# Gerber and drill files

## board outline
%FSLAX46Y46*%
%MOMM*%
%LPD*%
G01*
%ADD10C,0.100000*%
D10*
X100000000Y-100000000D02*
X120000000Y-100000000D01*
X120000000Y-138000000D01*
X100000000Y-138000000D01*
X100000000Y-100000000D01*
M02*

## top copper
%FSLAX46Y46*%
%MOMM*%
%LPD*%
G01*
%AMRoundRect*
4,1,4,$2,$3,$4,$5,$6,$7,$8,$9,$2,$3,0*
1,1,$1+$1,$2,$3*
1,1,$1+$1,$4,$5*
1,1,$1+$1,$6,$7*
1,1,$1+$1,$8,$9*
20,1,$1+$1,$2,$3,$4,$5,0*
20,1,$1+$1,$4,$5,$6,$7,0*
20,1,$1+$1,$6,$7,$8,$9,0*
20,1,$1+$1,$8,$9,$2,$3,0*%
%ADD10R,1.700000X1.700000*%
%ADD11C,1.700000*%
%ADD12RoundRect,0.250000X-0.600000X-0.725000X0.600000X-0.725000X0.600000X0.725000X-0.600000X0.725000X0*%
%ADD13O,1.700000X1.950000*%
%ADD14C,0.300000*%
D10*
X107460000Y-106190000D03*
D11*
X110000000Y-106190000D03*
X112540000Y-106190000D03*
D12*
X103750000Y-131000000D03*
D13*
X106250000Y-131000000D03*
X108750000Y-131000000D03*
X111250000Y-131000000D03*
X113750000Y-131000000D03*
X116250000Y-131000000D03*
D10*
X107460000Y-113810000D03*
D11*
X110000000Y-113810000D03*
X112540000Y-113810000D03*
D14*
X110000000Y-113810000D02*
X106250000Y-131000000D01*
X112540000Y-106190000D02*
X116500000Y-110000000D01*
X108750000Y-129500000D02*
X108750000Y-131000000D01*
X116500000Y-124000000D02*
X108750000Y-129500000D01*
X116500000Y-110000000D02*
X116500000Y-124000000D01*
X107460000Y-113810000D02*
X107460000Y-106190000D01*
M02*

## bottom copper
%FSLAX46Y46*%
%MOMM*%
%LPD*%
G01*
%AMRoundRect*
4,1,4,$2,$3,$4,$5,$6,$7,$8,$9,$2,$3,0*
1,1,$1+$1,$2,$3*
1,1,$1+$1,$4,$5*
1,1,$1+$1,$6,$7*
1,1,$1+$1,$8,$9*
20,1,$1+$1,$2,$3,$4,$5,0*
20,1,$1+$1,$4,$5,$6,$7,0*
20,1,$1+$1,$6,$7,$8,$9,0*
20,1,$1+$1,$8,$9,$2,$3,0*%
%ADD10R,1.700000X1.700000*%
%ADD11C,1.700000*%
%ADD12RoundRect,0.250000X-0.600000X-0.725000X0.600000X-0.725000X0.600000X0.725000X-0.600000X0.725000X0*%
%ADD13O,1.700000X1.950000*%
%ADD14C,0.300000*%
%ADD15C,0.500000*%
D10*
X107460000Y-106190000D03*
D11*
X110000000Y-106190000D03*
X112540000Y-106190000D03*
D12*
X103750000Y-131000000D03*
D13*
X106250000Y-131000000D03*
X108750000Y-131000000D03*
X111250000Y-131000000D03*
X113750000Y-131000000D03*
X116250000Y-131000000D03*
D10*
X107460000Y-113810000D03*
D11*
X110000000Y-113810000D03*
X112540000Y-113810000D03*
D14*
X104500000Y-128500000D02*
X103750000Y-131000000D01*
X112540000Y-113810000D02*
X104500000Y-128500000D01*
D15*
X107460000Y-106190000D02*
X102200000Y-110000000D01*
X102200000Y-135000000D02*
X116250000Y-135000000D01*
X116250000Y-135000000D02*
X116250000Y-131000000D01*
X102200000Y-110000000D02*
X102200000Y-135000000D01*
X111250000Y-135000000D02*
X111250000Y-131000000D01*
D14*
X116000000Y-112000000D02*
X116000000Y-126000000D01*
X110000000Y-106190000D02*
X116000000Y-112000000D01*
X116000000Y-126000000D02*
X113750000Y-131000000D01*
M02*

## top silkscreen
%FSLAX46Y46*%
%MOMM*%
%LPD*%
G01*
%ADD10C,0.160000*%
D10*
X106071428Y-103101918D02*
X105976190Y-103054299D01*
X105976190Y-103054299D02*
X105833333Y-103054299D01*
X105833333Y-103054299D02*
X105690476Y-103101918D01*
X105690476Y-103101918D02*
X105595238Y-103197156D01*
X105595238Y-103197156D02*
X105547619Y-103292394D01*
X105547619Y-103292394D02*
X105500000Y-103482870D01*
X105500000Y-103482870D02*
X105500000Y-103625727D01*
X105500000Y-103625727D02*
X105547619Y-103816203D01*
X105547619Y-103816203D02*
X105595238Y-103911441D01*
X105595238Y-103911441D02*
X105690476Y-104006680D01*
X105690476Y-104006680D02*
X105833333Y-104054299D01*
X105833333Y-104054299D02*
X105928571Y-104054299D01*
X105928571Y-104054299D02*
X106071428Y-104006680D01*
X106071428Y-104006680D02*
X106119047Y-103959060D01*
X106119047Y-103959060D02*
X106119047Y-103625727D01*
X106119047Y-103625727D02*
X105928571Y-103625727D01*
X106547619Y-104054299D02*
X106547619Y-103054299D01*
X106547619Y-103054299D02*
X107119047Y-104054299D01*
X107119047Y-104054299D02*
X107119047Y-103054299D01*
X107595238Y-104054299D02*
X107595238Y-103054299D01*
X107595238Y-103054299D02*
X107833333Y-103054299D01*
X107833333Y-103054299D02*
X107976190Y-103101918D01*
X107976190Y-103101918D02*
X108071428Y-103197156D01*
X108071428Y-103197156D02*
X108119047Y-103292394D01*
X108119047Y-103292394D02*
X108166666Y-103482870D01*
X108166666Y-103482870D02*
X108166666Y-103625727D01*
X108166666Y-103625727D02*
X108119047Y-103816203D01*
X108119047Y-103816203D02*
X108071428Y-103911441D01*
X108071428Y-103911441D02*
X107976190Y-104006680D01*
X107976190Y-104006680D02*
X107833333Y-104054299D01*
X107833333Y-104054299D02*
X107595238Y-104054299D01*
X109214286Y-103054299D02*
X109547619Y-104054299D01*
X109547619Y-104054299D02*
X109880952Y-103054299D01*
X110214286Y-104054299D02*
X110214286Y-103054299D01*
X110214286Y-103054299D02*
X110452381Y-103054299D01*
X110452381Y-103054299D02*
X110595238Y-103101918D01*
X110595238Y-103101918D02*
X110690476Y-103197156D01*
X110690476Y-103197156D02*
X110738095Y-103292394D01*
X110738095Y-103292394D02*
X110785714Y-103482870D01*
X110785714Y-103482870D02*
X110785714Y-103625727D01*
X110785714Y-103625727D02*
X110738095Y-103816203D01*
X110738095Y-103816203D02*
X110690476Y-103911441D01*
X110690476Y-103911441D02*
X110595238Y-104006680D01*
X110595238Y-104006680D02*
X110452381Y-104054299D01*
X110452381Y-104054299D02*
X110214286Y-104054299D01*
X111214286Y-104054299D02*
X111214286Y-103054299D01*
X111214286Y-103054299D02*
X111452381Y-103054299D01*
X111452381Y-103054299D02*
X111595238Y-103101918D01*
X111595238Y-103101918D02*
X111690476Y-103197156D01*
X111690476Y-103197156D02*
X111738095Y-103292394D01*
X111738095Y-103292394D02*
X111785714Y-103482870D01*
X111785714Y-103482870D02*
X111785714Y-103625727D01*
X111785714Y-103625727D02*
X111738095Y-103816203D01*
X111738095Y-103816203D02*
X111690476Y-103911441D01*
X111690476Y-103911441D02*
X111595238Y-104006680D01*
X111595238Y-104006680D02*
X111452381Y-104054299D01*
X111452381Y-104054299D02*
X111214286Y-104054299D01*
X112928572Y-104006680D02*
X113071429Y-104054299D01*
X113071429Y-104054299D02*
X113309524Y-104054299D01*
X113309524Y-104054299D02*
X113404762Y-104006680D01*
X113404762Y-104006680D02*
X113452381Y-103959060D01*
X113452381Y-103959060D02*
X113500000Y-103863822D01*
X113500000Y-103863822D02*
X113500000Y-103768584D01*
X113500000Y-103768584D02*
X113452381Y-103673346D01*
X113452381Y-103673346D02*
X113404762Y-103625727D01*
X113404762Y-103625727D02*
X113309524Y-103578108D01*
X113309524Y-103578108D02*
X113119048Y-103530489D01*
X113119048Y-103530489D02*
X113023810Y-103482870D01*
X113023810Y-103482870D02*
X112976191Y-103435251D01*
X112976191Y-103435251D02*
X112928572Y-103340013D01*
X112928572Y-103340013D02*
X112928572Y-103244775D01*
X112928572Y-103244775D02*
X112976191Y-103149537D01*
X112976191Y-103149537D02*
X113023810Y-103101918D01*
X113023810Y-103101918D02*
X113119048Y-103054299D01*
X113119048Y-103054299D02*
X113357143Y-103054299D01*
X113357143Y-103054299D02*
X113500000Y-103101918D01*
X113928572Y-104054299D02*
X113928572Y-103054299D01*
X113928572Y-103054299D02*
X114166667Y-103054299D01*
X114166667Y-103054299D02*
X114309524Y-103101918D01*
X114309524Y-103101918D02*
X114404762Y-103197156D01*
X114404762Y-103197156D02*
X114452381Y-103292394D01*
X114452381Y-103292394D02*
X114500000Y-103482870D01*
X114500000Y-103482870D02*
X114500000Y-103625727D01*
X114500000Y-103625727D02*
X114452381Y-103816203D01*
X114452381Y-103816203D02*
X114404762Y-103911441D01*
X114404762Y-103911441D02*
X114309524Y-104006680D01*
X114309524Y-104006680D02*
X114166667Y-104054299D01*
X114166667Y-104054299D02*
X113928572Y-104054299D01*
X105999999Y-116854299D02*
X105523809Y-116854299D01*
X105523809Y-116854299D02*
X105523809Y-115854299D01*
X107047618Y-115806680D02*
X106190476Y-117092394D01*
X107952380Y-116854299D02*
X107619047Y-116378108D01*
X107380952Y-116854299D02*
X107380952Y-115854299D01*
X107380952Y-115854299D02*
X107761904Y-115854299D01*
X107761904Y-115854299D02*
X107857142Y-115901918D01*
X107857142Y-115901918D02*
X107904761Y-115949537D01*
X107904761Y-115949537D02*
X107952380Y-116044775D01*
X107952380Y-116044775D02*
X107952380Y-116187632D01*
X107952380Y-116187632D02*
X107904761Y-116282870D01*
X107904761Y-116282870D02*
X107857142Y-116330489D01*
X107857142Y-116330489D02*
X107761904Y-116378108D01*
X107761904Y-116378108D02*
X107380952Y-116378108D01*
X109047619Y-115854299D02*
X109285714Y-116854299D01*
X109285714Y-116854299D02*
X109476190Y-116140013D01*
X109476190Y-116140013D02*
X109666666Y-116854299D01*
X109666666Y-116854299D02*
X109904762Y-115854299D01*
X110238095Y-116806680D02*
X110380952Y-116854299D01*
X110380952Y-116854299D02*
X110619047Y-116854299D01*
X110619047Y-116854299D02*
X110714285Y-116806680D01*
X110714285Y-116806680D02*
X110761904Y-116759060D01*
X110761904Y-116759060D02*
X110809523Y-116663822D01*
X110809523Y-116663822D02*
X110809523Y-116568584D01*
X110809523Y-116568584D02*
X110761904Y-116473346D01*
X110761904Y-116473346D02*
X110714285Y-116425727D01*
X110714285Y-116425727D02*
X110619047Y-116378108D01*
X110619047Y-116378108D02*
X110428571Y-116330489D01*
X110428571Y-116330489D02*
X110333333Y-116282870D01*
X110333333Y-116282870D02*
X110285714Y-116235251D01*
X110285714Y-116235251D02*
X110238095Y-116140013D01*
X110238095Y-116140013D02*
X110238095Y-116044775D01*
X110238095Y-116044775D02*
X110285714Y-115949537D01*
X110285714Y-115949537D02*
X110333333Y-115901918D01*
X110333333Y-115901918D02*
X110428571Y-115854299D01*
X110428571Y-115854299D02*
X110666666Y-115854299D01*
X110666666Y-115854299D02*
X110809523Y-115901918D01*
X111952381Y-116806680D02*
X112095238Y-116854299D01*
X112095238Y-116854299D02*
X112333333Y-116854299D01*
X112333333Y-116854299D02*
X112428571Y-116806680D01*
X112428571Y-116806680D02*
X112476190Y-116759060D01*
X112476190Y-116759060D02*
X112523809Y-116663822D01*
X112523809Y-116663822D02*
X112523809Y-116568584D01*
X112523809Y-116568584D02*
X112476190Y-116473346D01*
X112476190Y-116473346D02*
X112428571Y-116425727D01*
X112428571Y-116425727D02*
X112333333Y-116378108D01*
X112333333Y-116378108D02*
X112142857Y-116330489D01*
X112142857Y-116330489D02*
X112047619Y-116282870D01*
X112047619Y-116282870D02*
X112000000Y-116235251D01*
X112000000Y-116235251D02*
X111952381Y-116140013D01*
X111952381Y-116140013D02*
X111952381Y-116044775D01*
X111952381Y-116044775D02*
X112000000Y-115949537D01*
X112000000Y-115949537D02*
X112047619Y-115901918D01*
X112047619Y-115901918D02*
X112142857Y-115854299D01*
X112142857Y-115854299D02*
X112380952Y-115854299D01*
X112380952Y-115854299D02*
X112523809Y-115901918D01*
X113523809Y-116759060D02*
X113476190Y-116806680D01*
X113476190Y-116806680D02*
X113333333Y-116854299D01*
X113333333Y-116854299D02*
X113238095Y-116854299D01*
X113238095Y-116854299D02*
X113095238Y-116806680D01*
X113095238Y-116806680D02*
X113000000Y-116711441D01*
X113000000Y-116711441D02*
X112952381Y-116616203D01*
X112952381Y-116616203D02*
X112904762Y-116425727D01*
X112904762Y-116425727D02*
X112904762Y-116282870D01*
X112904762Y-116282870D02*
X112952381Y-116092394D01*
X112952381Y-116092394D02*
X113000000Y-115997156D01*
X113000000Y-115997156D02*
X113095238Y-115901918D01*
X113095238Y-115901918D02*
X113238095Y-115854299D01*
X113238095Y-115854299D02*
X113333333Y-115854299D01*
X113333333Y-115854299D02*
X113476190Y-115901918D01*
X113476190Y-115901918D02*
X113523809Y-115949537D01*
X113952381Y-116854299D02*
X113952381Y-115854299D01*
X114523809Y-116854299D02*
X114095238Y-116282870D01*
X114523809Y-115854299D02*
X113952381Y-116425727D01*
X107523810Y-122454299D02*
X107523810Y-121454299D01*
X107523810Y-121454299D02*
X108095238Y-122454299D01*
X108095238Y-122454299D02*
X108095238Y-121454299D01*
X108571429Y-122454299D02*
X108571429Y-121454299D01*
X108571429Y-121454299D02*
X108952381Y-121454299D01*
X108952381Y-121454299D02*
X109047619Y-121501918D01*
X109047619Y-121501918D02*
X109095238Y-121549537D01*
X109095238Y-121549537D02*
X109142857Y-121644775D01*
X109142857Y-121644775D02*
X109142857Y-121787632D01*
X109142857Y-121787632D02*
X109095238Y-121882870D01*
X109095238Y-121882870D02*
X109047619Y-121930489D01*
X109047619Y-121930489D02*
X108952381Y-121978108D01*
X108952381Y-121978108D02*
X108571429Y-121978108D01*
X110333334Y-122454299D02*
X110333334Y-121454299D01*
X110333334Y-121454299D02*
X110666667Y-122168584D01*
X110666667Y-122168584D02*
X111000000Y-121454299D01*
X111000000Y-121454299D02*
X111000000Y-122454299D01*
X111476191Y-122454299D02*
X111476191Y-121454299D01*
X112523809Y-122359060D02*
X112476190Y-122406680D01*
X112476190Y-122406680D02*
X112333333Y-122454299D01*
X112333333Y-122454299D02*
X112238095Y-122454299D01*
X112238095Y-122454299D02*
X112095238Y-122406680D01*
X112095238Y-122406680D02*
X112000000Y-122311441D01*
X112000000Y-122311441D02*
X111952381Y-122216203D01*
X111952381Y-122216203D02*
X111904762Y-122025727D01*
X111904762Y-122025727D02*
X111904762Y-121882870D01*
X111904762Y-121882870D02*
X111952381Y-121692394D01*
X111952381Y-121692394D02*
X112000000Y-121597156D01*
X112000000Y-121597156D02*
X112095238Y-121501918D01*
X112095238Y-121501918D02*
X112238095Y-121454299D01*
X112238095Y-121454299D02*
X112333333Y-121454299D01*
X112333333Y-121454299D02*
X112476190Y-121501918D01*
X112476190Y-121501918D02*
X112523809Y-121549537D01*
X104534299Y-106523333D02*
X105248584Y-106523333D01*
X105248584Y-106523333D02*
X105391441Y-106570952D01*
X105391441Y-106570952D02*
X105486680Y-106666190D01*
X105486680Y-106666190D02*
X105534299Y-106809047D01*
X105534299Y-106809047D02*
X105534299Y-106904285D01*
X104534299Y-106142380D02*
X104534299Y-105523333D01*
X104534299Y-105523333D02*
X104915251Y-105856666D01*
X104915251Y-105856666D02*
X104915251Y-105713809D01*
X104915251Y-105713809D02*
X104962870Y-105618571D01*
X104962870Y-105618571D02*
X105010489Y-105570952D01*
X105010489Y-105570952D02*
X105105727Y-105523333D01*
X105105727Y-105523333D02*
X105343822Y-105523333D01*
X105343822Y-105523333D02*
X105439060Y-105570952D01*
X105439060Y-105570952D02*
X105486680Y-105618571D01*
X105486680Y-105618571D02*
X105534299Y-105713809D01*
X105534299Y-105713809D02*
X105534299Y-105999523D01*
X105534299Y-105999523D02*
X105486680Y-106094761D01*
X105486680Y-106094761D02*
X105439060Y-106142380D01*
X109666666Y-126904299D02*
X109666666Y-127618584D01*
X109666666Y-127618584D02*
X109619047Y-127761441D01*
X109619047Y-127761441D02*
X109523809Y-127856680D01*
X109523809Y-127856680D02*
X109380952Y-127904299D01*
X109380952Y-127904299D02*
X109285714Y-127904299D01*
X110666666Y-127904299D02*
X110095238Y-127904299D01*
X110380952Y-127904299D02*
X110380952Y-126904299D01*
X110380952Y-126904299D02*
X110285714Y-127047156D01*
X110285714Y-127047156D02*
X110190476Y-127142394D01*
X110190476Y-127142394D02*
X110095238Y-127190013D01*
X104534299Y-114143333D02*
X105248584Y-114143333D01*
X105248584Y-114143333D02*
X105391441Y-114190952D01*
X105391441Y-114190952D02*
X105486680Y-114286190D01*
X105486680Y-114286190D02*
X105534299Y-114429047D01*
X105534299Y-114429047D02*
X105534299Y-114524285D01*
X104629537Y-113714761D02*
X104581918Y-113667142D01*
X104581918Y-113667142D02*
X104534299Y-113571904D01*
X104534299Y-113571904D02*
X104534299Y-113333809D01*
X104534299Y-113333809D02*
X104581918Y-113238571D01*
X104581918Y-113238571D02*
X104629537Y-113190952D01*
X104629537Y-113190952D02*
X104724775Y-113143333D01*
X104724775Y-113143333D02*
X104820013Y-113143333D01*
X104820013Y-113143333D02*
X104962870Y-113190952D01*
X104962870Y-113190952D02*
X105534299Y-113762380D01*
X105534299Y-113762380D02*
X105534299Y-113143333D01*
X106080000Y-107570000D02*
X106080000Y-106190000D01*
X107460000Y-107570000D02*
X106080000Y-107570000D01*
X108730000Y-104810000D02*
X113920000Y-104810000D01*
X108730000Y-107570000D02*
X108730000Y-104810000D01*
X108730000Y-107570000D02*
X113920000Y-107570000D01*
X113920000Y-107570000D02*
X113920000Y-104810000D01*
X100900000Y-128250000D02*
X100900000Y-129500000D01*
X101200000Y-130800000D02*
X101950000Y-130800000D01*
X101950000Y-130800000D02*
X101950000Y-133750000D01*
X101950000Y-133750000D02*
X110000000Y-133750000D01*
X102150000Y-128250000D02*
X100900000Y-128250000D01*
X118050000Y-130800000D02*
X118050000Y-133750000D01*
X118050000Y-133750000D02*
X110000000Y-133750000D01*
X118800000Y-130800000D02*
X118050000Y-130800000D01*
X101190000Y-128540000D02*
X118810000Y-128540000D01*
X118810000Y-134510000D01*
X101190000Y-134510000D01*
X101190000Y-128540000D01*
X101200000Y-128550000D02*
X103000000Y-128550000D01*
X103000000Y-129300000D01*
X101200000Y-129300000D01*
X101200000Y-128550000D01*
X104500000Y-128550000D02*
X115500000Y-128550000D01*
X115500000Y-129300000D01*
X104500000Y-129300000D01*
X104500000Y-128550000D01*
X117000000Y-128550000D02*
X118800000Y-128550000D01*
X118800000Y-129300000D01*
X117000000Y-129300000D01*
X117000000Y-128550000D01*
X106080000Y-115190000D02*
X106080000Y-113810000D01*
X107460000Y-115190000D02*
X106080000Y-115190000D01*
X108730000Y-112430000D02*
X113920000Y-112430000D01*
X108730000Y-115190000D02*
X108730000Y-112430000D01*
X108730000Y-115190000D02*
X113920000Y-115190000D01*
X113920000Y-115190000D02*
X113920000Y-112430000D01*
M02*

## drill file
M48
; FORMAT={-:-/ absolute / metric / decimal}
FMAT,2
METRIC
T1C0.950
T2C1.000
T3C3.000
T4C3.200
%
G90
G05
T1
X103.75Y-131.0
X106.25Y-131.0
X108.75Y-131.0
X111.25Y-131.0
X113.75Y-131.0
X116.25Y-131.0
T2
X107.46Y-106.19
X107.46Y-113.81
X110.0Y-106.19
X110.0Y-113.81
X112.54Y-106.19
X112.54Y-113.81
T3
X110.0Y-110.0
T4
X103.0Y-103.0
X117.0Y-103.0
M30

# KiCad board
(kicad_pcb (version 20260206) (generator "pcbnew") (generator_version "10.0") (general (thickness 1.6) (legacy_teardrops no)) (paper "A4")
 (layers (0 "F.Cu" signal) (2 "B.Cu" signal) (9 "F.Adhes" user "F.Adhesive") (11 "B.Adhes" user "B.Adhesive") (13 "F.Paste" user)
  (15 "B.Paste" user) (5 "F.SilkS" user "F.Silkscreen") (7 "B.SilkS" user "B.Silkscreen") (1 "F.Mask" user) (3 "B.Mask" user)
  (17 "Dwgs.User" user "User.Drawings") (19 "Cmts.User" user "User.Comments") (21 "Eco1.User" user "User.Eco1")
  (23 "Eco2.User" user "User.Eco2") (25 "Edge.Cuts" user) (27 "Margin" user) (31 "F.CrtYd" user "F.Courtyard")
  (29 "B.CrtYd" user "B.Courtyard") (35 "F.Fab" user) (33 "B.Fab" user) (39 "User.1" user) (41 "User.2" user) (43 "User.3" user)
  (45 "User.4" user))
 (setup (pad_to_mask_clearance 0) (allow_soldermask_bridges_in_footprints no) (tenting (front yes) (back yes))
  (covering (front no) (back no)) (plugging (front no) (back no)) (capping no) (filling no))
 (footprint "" (layer "F.Cu") (at 110 110)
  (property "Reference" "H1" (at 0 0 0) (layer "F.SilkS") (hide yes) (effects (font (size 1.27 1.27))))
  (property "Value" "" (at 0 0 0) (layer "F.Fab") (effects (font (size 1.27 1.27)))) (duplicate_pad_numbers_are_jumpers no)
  (pad "" np_thru_hole circle (at 0 0) (size 3 3) (drill 3) (layers "*.Cu" "*.Mask")))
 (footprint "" (layer "F.Cu") (at 117 103)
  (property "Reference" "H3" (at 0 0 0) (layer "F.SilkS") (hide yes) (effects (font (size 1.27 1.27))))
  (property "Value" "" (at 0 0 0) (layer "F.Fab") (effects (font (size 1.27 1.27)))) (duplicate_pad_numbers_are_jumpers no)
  (pad "" np_thru_hole circle (at 0 0) (size 3.2 3.2) (drill 3.2) (layers "*.Cu" "*.Mask")))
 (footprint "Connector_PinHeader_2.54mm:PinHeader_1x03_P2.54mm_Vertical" (layer "F.Cu") (at 107.46 106.19 90)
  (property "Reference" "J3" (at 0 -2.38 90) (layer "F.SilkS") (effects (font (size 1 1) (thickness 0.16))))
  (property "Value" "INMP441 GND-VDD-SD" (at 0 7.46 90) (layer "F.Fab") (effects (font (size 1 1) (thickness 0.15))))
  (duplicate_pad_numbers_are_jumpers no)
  (fp_line (start -1.38 -1.38) (end 0 -1.38) (stroke (width 0.16) (type solid)) (layer "F.SilkS"))
  (fp_line (start -1.38 0) (end -1.38 -1.38) (stroke (width 0.16) (type solid)) (layer "F.SilkS"))
  (fp_line (start 1.38 1.27) (end 1.38 6.46) (stroke (width 0.16) (type solid)) (layer "F.SilkS"))
  (fp_line (start -1.38 1.27) (end 1.38 1.27) (stroke (width 0.16) (type solid)) (layer "F.SilkS"))
  (fp_line (start -1.38 1.27) (end -1.38 6.46) (stroke (width 0.16) (type solid)) (layer "F.SilkS"))
  (fp_line (start -1.38 6.46) (end 1.38 6.46) (stroke (width 0.16) (type solid)) (layer "F.SilkS"))
  (pad "1" thru_hole rect (at 0 0 90) (size 1.7 1.7) (drill 1) (layers "*.Cu" "*.Mask") (remove_unused_layers no) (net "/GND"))
  (pad "2" thru_hole circle (at 0 2.54 90) (size 1.7 1.7) (drill 1) (layers "*.Cu" "*.Mask") (remove_unused_layers no) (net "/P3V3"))
  (pad "3" thru_hole circle (at 0 5.08 90) (size 1.7 1.7) (drill 1) (layers "*.Cu" "*.Mask") (remove_unused_layers no) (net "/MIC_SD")))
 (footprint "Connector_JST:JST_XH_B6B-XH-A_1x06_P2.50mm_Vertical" (layer "F.Cu") (at 103.75 131)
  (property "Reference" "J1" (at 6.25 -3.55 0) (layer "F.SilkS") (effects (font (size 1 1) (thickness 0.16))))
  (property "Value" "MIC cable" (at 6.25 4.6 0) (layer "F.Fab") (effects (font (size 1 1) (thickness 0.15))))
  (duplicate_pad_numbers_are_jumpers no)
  (fp_line (start -2.85 -2.75) (end -2.85 -1.5) (stroke (width 0.16) (type solid)) (layer "F.SilkS"))
  (fp_line (start -2.55 -0.2) (end -1.8 -0.2) (stroke (width 0.16) (type solid)) (layer "F.SilkS"))
  (fp_line (start -1.8 -0.2) (end -1.8 2.75) (stroke (width 0.16) (type solid)) (layer "F.SilkS"))
  (fp_line (start -1.8 2.75) (end 6.25 2.75) (stroke (width 0.16) (type solid)) (layer "F.SilkS"))
  (fp_line (start -1.6 -2.75) (end -2.85 -2.75) (stroke (width 0.16) (type solid)) (layer "F.SilkS"))
  (fp_line (start 14.3 -0.2) (end 14.3 2.75) (stroke (width 0.16) (type solid)) (layer "F.SilkS"))
  (fp_line (start 14.3 2.75) (end 6.25 2.75) (stroke (width 0.16) (type solid)) (layer "F.SilkS"))
  (fp_line (start 15.05 -0.2) (end 14.3 -0.2) (stroke (width 0.16) (type solid)) (layer "F.SilkS"))
  (fp_rect (start -2.56 -2.46) (end 15.06 3.51) (stroke (width 0.16) (type solid)) (fill no) (layer "F.SilkS"))
  (fp_rect (start -2.55 -2.45) (end -0.75 -1.7) (stroke (width 0.16) (type solid)) (fill no) (layer "F.SilkS"))
  (fp_rect (start 0.75 -2.45) (end 11.75 -1.7) (stroke (width 0.16) (type solid)) (fill no) (layer "F.SilkS"))
  (fp_rect (start 13.25 -2.45) (end 15.05 -1.7) (stroke (width 0.16) (type solid)) (fill no) (layer "F.SilkS"))
  (pad "1" thru_hole roundrect (at 0 0) (size 1.7 1.95) (drill 0.95) (layers "*.Cu" "*.Mask") (remove_unused_layers no)
   (roundrect_rratio 0.147059) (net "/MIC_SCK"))
  (pad "2" thru_hole oval (at 2.5 0) (size 1.7 1.95) (drill 0.95) (layers "*.Cu" "*.Mask") (remove_unused_layers no) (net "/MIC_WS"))
  (pad "3" thru_hole oval (at 5 0) (size 1.7 1.95) (drill 0.95) (layers "*.Cu" "*.Mask") (remove_unused_layers no) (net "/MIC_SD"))
  (pad "4" thru_hole oval (at 7.5 0) (size 1.7 1.95) (drill 0.95) (layers "*.Cu" "*.Mask") (remove_unused_layers no) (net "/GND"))
  (pad "5" thru_hole oval (at 10 0) (size 1.7 1.95) (drill 0.95) (layers "*.Cu" "*.Mask") (remove_unused_layers no) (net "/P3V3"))
  (pad "6" thru_hole oval (at 12.5 0) (size 1.7 1.95) (drill 0.95) (layers "*.Cu" "*.Mask") (remove_unused_layers no) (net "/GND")))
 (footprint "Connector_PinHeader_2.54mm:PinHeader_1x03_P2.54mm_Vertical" (layer "F.Cu") (at 107.46 113.81 90)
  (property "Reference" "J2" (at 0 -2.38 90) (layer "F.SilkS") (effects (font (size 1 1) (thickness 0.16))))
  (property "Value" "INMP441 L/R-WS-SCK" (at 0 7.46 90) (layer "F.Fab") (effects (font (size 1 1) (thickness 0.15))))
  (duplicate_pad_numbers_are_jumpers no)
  (fp_line (start -1.38 -1.38) (end 0 -1.38) (stroke (width 0.16) (type solid)) (layer "F.SilkS"))
  (fp_line (start -1.38 0) (end -1.38 -1.38) (stroke (width 0.16) (type solid)) (layer "F.SilkS"))
  (fp_line (start 1.38 1.27) (end 1.38 6.46) (stroke (width 0.16) (type solid)) (layer "F.SilkS"))
  (fp_line (start -1.38 1.27) (end 1.38 1.27) (stroke (width 0.16) (type solid)) (layer "F.SilkS"))
  (fp_line (start -1.38 1.27) (end -1.38 6.46) (stroke (width 0.16) (type solid)) (layer "F.SilkS"))
  (fp_line (start -1.38 6.46) (end 1.38 6.46) (stroke (width 0.16) (type solid)) (layer "F.SilkS"))
  (pad "1" thru_hole rect (at 0 0 90) (size 1.7 1.7) (drill 1) (layers "*.Cu" "*.Mask") (remove_unused_layers no) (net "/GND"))
  (pad "2" thru_hole circle (at 0 2.54 90) (size 1.7 1.7) (drill 1) (layers "*.Cu" "*.Mask") (remove_unused_layers no) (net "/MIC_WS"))
  (pad "3" thru_hole circle (at 0 5.08 90) (size 1.7 1.7) (drill 1) (layers "*.Cu" "*.Mask") (remove_unused_layers no) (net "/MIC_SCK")))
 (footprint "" (layer "F.Cu") (at 103 103)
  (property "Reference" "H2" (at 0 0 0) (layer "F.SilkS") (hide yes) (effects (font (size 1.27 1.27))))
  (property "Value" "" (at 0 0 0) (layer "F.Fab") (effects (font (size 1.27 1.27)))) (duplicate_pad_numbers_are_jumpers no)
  (pad "" np_thru_hole circle (at 0 0) (size 3.2 3.2) (drill 3.2) (layers "*.Cu" "*.Mask")))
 (gr_rect (start 100 100) (end 120 138) (stroke (width 0.1) (type default)) (fill no) (layer "Edge.Cuts"))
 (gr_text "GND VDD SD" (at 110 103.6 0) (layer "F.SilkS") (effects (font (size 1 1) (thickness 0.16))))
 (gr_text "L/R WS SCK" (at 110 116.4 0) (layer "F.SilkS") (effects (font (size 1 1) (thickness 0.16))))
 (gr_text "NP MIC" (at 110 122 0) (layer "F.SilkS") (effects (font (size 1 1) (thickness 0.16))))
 (segment (start 104.5 128.5) (end 103.75 131) (width 0.3) (layer "B.Cu") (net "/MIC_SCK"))
 (segment (start 112.54 113.81) (end 104.5 128.5) (width 0.3) (layer "B.Cu") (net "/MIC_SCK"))
 (segment (start 110 113.81) (end 106.25 131) (width 0.3) (layer "F.Cu") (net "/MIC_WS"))
 (segment (start 112.54 106.19) (end 116.5 110) (width 0.3) (layer "F.Cu") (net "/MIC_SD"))
 (segment (start 108.75 129.5) (end 108.75 131) (width 0.3) (layer "F.Cu") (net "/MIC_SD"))
 (segment (start 116.5 124) (end 108.75 129.5) (width 0.3) (layer "F.Cu") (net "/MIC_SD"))
 (segment (start 116.5 110) (end 116.5 124) (width 0.3) (layer "F.Cu") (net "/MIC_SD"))
 (segment (start 107.46 113.81) (end 107.46 106.19) (width 0.3) (layer "F.Cu") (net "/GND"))
 (segment (start 107.46 106.19) (end 102.2 110) (width 0.5) (layer "B.Cu") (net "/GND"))
 (segment (start 102.2 135) (end 116.25 135) (width 0.5) (layer "B.Cu") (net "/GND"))
 (segment (start 116.25 135) (end 116.25 131) (width 0.5) (layer "B.Cu") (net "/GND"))
 (segment (start 102.2 110) (end 102.2 135) (width 0.5) (layer "B.Cu") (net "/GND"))
 (segment (start 111.25 135) (end 111.25 131) (width 0.5) (layer "B.Cu") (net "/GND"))
 (segment (start 116 112) (end 116 126) (width 0.3) (layer "B.Cu") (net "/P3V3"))
 (segment (start 110 106.19) (end 116 112) (width 0.3) (layer "B.Cu") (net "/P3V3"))
 (segment (start 116 126) (end 113.75 131) (width 0.3) (layer "B.Cu") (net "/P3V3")))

